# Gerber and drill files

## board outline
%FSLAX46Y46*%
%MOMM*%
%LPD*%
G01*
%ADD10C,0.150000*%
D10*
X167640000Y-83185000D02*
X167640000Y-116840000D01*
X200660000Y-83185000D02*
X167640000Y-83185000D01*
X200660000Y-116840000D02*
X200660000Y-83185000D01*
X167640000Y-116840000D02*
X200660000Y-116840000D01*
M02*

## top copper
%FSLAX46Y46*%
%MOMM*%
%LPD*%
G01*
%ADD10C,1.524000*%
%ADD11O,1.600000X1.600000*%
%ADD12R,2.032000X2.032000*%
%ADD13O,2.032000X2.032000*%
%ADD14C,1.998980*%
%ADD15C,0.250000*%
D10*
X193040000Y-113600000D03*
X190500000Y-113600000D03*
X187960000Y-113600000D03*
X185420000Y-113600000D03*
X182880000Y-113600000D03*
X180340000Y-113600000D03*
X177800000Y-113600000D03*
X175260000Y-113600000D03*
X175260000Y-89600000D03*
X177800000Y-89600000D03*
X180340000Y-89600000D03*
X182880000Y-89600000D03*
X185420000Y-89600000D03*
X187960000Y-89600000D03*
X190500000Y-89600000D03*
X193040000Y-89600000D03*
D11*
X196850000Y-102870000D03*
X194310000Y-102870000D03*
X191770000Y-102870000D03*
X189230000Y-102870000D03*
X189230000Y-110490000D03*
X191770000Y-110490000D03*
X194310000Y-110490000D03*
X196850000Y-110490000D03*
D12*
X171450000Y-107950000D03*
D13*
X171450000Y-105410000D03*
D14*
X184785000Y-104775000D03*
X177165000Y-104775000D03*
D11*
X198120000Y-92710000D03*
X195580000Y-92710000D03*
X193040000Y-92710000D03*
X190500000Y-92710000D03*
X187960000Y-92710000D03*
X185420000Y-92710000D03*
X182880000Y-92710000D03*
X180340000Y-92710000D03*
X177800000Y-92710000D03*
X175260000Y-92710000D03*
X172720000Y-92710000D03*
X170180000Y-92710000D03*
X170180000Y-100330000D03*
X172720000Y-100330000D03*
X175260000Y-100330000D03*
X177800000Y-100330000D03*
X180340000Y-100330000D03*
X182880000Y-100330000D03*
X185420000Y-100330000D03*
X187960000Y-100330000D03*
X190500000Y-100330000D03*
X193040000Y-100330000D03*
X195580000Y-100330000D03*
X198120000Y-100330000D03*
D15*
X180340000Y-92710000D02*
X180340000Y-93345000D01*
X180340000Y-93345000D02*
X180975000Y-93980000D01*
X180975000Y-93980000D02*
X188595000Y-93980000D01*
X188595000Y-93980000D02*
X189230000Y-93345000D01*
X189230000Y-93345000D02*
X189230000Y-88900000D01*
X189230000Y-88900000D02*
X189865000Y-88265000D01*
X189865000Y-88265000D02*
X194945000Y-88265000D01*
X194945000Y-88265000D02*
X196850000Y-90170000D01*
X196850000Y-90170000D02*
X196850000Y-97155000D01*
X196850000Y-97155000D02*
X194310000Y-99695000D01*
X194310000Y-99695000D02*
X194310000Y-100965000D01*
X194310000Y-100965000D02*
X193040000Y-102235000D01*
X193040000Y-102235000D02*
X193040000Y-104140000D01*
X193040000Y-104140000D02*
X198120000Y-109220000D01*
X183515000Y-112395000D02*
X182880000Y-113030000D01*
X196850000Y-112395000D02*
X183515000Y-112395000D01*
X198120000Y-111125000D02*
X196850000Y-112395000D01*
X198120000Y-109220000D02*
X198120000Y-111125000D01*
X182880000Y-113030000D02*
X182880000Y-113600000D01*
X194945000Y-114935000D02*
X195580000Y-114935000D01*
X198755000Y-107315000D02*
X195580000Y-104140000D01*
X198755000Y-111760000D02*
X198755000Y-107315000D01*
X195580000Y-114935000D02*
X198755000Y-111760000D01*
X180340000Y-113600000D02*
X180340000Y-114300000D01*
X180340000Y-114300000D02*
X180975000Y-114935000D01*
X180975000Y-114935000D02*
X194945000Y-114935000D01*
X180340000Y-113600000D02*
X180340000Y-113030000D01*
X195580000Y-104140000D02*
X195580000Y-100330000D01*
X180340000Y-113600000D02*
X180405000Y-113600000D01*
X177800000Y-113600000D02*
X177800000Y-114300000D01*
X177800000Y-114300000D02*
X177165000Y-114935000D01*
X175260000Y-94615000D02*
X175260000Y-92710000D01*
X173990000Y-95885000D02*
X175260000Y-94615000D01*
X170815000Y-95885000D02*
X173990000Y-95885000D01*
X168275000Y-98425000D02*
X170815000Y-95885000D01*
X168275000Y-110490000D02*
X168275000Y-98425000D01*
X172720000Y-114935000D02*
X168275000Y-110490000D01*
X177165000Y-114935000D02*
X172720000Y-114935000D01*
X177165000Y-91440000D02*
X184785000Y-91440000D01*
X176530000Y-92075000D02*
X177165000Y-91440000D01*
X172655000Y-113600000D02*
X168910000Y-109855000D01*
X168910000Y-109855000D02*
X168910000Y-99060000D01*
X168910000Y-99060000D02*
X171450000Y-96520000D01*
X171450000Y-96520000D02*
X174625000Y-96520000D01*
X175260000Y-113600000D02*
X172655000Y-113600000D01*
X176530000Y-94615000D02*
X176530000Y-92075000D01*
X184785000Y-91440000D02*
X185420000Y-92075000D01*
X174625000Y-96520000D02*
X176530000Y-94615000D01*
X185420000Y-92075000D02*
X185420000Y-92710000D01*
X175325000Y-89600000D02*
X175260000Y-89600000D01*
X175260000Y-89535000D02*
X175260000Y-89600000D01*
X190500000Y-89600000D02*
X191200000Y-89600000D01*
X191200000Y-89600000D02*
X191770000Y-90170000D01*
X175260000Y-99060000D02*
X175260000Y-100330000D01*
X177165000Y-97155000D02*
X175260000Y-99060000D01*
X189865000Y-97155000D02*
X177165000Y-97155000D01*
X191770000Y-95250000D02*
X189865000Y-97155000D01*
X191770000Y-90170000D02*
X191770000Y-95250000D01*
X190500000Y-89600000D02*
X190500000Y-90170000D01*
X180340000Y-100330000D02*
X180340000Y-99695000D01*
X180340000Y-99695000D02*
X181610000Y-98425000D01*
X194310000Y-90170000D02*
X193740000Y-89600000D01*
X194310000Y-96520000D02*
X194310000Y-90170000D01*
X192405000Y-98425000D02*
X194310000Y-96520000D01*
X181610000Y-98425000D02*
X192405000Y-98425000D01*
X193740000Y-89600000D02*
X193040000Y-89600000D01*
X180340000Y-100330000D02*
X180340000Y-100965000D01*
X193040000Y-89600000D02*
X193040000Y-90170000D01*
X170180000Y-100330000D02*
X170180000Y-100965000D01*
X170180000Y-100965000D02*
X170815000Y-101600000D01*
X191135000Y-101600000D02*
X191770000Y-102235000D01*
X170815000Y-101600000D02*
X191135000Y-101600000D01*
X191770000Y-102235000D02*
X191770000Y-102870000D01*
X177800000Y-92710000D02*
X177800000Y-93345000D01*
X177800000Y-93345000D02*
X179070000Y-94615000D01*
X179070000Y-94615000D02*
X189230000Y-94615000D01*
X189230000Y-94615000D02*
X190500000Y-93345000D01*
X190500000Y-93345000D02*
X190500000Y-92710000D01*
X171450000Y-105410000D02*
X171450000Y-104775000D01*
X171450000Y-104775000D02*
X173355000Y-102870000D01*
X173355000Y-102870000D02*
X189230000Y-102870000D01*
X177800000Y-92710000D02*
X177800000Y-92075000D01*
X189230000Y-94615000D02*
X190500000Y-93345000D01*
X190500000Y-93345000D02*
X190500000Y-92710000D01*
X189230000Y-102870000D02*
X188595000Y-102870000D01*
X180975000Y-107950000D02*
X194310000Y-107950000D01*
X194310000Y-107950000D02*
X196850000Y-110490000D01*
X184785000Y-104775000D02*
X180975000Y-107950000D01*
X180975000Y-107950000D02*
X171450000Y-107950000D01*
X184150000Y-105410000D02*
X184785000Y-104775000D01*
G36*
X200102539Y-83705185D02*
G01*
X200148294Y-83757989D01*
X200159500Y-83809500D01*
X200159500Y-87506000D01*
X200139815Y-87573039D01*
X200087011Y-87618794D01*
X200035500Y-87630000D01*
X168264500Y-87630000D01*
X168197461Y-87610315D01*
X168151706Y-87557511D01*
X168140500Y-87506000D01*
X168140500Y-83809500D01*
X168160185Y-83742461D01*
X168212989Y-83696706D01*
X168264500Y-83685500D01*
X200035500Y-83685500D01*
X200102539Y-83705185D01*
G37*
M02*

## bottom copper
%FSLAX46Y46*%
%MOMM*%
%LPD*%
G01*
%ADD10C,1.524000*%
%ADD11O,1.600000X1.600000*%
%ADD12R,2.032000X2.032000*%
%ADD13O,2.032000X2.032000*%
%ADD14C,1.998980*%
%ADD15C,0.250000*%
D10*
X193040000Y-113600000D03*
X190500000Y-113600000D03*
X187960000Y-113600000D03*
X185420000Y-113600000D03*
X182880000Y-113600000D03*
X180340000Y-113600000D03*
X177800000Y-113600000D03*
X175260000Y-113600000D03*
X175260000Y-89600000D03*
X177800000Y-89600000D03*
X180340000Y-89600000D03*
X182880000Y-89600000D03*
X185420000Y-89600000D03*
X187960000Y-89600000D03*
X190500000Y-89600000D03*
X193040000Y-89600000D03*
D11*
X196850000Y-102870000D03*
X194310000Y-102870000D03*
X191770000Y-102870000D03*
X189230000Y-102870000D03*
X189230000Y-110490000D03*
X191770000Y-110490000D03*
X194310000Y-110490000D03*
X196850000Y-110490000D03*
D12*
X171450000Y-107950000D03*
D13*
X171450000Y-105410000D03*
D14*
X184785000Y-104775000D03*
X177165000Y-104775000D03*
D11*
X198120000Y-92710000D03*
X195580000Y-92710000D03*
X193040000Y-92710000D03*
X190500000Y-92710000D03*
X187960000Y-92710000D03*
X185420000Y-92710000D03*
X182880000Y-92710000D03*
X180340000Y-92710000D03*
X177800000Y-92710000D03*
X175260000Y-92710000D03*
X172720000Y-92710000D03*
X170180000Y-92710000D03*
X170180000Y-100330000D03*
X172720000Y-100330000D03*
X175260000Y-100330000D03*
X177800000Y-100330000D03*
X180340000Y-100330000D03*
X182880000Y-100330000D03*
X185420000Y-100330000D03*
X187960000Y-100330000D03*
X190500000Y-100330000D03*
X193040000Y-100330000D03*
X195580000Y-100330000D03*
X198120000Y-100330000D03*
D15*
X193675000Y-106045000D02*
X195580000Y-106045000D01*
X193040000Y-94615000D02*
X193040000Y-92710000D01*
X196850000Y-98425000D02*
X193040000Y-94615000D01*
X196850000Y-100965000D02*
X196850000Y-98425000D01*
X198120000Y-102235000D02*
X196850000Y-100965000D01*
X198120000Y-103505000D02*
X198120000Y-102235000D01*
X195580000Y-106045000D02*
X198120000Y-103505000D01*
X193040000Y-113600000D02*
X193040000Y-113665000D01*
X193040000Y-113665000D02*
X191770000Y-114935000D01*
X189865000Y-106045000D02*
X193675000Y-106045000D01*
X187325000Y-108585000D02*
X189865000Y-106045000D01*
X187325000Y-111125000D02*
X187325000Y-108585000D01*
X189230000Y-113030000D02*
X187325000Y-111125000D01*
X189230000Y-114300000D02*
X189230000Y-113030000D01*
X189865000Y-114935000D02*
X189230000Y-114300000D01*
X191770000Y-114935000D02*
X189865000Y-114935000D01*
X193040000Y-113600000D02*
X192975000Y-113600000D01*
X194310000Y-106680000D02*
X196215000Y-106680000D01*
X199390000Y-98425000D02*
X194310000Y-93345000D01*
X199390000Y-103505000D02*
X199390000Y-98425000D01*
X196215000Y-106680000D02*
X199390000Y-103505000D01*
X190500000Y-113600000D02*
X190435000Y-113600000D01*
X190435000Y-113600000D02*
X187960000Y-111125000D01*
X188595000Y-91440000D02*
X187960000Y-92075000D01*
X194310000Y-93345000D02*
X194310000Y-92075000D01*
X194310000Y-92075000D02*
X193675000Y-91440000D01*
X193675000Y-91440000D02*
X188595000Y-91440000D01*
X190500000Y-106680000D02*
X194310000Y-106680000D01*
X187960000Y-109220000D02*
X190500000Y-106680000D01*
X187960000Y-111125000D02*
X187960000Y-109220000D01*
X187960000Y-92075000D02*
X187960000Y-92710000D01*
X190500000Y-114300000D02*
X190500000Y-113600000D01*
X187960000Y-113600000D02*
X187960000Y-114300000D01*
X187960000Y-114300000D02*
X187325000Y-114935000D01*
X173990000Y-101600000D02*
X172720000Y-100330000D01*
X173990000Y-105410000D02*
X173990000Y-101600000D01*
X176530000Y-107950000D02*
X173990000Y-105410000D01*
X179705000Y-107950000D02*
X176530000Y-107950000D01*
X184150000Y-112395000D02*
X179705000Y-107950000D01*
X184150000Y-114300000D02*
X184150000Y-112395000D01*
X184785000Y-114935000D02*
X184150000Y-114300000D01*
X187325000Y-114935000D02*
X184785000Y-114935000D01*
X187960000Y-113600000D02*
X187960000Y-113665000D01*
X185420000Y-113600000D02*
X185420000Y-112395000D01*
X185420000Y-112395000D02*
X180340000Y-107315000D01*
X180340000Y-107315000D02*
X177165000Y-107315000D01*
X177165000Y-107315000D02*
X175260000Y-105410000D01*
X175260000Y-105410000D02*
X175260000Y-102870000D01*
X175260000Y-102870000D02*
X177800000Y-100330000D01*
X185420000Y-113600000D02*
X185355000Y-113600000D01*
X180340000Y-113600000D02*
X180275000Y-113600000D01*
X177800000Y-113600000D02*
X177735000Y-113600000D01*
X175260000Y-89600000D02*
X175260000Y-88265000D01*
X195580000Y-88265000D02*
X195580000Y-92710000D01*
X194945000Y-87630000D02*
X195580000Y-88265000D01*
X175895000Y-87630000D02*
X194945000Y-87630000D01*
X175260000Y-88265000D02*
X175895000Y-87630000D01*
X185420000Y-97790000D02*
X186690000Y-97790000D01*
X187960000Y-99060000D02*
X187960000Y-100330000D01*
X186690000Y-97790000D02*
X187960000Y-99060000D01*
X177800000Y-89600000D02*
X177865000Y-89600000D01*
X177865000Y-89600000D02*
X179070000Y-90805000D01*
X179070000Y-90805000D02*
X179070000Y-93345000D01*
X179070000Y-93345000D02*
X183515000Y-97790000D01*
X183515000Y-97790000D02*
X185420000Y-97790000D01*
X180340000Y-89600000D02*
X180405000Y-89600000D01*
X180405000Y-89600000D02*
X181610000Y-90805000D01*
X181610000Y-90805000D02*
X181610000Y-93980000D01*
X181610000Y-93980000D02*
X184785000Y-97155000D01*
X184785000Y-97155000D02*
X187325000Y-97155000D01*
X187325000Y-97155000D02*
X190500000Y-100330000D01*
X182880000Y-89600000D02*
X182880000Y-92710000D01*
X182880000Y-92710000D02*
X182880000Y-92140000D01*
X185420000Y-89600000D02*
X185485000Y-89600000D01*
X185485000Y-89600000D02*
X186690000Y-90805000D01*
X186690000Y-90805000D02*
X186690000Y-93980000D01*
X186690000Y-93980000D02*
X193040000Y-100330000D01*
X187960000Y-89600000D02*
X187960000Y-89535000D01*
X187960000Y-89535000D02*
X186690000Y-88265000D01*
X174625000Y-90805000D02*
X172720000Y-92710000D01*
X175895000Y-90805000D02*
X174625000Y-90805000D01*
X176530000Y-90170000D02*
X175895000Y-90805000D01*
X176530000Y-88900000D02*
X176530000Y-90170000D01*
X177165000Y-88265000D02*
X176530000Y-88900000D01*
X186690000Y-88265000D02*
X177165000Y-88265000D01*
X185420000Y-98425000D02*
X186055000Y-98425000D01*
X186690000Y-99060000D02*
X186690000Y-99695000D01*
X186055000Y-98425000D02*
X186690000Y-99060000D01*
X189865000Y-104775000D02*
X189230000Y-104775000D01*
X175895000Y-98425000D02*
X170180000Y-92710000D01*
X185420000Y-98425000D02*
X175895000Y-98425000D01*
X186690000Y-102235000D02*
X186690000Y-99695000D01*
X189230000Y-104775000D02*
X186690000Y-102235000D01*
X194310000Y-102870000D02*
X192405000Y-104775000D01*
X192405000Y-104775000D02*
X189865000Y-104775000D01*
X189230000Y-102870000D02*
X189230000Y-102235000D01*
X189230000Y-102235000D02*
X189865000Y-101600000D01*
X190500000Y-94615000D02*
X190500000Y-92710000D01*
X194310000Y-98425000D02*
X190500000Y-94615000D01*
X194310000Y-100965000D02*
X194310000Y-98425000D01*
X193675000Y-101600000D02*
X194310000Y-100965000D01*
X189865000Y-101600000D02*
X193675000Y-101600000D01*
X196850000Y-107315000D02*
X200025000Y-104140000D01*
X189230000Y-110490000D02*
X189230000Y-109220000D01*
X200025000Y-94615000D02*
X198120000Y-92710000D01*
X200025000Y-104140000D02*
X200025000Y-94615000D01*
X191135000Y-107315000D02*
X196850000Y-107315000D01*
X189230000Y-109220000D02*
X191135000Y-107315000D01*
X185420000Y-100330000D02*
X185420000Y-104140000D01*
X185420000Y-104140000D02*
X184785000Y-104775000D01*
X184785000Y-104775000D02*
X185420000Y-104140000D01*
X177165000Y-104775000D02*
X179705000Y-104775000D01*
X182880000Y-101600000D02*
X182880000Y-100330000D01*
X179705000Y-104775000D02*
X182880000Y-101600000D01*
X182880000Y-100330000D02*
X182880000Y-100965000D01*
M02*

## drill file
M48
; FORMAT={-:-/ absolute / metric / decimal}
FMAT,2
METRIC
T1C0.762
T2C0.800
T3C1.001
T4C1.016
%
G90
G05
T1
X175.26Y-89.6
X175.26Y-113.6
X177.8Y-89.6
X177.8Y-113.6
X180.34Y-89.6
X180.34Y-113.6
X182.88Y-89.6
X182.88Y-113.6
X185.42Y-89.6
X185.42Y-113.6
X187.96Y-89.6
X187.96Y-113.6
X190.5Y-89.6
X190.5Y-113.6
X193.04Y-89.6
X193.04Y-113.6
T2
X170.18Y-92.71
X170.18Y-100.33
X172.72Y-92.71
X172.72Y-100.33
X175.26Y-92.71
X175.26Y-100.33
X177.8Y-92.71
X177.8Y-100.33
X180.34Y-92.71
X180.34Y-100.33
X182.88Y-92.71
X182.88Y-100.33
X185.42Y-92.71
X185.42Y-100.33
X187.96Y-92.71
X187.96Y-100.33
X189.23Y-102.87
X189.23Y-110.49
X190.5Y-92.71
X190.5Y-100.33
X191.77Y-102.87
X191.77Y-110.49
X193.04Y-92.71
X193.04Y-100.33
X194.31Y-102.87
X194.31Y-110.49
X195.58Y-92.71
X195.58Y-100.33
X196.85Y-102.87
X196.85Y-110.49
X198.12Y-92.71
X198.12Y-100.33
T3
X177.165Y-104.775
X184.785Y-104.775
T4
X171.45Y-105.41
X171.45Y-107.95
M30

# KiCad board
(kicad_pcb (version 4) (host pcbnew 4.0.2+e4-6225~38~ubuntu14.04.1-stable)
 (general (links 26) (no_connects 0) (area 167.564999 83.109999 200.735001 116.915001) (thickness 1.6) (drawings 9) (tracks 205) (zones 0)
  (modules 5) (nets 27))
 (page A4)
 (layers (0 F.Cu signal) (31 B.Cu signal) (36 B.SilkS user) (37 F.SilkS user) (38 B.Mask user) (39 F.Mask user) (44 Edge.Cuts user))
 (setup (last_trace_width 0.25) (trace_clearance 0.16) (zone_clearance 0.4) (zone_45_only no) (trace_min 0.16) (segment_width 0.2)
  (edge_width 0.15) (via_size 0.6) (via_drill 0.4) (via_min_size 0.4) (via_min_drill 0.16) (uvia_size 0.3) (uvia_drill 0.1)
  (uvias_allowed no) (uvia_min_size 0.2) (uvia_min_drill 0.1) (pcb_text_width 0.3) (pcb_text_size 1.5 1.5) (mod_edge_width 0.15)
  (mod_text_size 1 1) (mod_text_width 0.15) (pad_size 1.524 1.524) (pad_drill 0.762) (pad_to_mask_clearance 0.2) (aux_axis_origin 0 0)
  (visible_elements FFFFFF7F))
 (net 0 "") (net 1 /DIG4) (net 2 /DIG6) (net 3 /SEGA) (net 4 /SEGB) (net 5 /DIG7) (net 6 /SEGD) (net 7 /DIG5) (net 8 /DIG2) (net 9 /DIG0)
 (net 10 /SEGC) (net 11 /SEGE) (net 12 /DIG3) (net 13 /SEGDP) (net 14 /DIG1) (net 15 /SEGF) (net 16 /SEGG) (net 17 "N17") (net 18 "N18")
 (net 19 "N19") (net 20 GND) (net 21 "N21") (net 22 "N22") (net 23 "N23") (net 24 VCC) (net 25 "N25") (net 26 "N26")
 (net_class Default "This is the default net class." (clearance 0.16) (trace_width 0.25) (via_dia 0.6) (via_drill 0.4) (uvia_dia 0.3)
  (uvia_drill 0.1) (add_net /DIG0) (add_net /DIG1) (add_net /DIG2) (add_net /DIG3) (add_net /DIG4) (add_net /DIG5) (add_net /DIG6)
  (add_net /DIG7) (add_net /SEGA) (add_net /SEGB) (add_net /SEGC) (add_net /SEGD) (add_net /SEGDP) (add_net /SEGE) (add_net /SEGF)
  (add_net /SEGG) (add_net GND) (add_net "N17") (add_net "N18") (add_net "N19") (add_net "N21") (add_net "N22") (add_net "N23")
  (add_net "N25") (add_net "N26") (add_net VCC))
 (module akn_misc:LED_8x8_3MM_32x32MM (layer B.Cu) (at 184.15 101.6 90)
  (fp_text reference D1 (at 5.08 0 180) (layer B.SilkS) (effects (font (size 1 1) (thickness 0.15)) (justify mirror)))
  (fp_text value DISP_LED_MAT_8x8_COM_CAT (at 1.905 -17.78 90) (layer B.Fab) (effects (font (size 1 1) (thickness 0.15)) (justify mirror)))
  (pad 1 thru_hole circle (at -12 8.89 90) (size 1.524 1.524) (drill 0.762) (layers *.Cu *.Mask B.SilkS) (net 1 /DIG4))
  (pad 2 thru_hole circle (at -12 6.35 90) (size 1.524 1.524) (drill 0.762) (layers *.Cu *.Mask B.SilkS) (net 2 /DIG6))
  (pad 3 thru_hole circle (at -12 3.81 90) (size 1.524 1.524) (drill 0.762) (layers *.Cu *.Mask B.SilkS) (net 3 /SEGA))
  (pad 4 thru_hole circle (at -12 1.27 90) (size 1.524 1.524) (drill 0.762) (layers *.Cu *.Mask B.SilkS) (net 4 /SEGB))
  (pad 5 thru_hole circle (at -12 -1.27 90) (size 1.524 1.524) (drill 0.762) (layers *.Cu *.Mask B.SilkS) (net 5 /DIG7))
  (pad 6 thru_hole circle (at -12 -3.81 90) (size 1.524 1.524) (drill 0.762) (layers *.Cu *.Mask B.SilkS) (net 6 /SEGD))
  (pad 7 thru_hole circle (at -12 -6.35 90) (size 1.524 1.524) (drill 0.762) (layers *.Cu *.Mask B.SilkS) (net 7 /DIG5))
  (pad 8 thru_hole circle (at -12 -8.89 90) (size 1.524 1.524) (drill 0.762) (layers *.Cu *.Mask B.SilkS) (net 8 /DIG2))
  (pad 9 thru_hole circle (at 12 -8.89 90) (size 1.524 1.524) (drill 0.762) (layers *.Cu *.Mask B.SilkS) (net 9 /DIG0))
  (pad 10 thru_hole circle (at 12 -6.35 90) (size 1.524 1.524) (drill 0.762) (layers *.Cu *.Mask B.SilkS) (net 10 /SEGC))
  (pad 11 thru_hole circle (at 12 -3.81 90) (size 1.524 1.524) (drill 0.762) (layers *.Cu *.Mask B.SilkS) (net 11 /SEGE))
  (pad 12 thru_hole circle (at 12 -1.27 90) (size 1.524 1.524) (drill 0.762) (layers *.Cu *.Mask B.SilkS) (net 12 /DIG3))
  (pad 13 thru_hole circle (at 12 1.27 90) (size 1.524 1.524) (drill 0.762) (layers *.Cu *.Mask B.SilkS) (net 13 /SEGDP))
  (pad 14 thru_hole circle (at 12 3.81 90) (size 1.524 1.524) (drill 0.762) (layers *.Cu *.Mask B.SilkS) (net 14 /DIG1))
  (pad 15 thru_hole circle (at 12 6.35 90) (size 1.524 1.524) (drill 0.762) (layers *.Cu *.Mask B.SilkS) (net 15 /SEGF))
  (pad 16 thru_hole circle (at 12 8.89 90) (size 1.524 1.524) (drill 0.762) (layers *.Cu *.Mask B.SilkS) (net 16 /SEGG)))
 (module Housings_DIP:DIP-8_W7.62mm (layer F.Cu) (at 196.85 102.87 270)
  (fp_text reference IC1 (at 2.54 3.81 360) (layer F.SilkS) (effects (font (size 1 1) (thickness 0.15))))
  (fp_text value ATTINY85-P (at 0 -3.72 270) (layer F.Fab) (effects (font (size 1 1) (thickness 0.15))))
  (pad 1 thru_hole oval (at 0 0 270) (size 1.6 1.6) (drill 0.8) (layers *.Cu *.Mask F.SilkS) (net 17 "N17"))
  (pad 2 thru_hole oval (at 0 2.54 270) (size 1.6 1.6) (drill 0.8) (layers *.Cu *.Mask F.SilkS) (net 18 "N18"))
  (pad 3 thru_hole oval (at 0 5.08 270) (size 1.6 1.6) (drill 0.8) (layers *.Cu *.Mask F.SilkS) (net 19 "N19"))
  (pad 4 thru_hole oval (at 0 7.62 270) (size 1.6 1.6) (drill 0.8) (layers *.Cu *.Mask F.SilkS) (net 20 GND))
  (pad 5 thru_hole oval (at 7.62 7.62 270) (size 1.6 1.6) (drill 0.8) (layers *.Cu *.Mask F.SilkS) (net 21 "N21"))
  (pad 6 thru_hole oval (at 7.62 5.08 270) (size 1.6 1.6) (drill 0.8) (layers *.Cu *.Mask F.SilkS) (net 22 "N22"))
  (pad 7 thru_hole oval (at 7.62 2.54 270) (size 1.6 1.6) (drill 0.8) (layers *.Cu *.Mask F.SilkS) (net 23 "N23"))
  (pad 8 thru_hole oval (at 7.62 0 270) (size 1.6 1.6) (drill 0.8) (layers *.Cu *.Mask F.SilkS) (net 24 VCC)))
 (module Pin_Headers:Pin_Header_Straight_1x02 (layer F.Cu) (at 171.45 107.95 180)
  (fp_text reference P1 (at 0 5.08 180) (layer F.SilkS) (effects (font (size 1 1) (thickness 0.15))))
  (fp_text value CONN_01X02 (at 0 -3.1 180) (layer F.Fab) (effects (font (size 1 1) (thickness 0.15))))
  (pad 1 thru_hole rect (at 0 0 180) (size 2.032 2.032) (drill 1.016) (layers *.Cu *.Mask F.SilkS) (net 24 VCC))
  (pad 2 thru_hole oval (at 0 2.54 180) (size 2.032 2.032) (drill 1.016) (layers *.Cu *.Mask F.SilkS) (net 20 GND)))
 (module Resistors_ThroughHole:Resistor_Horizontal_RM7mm (layer F.Cu) (at 184.785 104.775 180)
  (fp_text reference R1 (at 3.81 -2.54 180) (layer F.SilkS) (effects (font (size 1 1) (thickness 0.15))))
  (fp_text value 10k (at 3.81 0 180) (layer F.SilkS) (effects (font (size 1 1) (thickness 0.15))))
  (pad 1 thru_hole circle (at 0 0 180) (size 1.99898 1.99898) (drill 1.00076) (layers *.Cu *.SilkS *.Mask) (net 24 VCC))
  (pad 2 thru_hole circle (at 7.62 0 180) (size 1.99898 1.99898) (drill 1.00076) (layers *.Cu *.SilkS *.Mask) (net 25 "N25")))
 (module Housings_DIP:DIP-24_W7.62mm (layer F.Cu) (at 198.12 92.71 270)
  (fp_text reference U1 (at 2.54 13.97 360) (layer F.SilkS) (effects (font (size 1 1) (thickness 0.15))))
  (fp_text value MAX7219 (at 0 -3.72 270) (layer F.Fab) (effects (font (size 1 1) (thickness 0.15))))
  (pad 1 thru_hole oval (at 0 0 270) (size 1.6 1.6) (drill 0.8) (layers *.Cu *.Mask F.SilkS) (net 21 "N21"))
  (pad 2 thru_hole oval (at 0 2.54 270) (size 1.6 1.6) (drill 0.8) (layers *.Cu *.Mask F.SilkS) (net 9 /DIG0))
  (pad 3 thru_hole oval (at 0 5.08 270) (size 1.6 1.6) (drill 0.8) (layers *.Cu *.Mask F.SilkS) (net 1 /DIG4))
  (pad 4 thru_hole oval (at 0 7.62 270) (size 1.6 1.6) (drill 0.8) (layers *.Cu *.Mask F.SilkS) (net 20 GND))
  (pad 5 thru_hole oval (at 0 10.16 270) (size 1.6 1.6) (drill 0.8) (layers *.Cu *.Mask F.SilkS) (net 2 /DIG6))
  (pad 6 thru_hole oval (at 0 12.7 270) (size 1.6 1.6) (drill 0.8) (layers *.Cu *.Mask F.SilkS) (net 8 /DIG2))
  (pad 7 thru_hole oval (at 0 15.24 270) (size 1.6 1.6) (drill 0.8) (layers *.Cu *.Mask F.SilkS) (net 12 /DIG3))
  (pad 8 thru_hole oval (at 0 17.78 270) (size 1.6 1.6) (drill 0.8) (layers *.Cu *.Mask F.SilkS) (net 5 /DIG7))
  (pad 9 thru_hole oval (at 0 20.32 270) (size 1.6 1.6) (drill 0.8) (layers *.Cu *.Mask F.SilkS) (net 20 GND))
  (pad 10 thru_hole oval (at 0 22.86 270) (size 1.6 1.6) (drill 0.8) (layers *.Cu *.Mask F.SilkS) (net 7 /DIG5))
  (pad 11 thru_hole oval (at 0 25.4 270) (size 1.6 1.6) (drill 0.8) (layers *.Cu *.Mask F.SilkS) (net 14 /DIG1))
  (pad 12 thru_hole oval (at 0 27.94 270) (size 1.6 1.6) (drill 0.8) (layers *.Cu *.Mask F.SilkS) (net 18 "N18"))
  (pad 13 thru_hole oval (at 7.62 27.94 270) (size 1.6 1.6) (drill 0.8) (layers *.Cu *.Mask F.SilkS) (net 19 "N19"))
  (pad 14 thru_hole oval (at 7.62 25.4 270) (size 1.6 1.6) (drill 0.8) (layers *.Cu *.Mask F.SilkS) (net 3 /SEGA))
  (pad 15 thru_hole oval (at 7.62 22.86 270) (size 1.6 1.6) (drill 0.8) (layers *.Cu *.Mask F.SilkS) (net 15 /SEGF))
  (pad 16 thru_hole oval (at 7.62 20.32 270) (size 1.6 1.6) (drill 0.8) (layers *.Cu *.Mask F.SilkS) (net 4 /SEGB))
  (pad 17 thru_hole oval (at 7.62 17.78 270) (size 1.6 1.6) (drill 0.8) (layers *.Cu *.Mask F.SilkS) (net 16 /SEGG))
  (pad 18 thru_hole oval (at 7.62 15.24 270) (size 1.6 1.6) (drill 0.8) (layers *.Cu *.Mask F.SilkS) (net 25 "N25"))
  (pad 19 thru_hole oval (at 7.62 12.7 270) (size 1.6 1.6) (drill 0.8) (layers *.Cu *.Mask F.SilkS) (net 24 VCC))
  (pad 20 thru_hole oval (at 7.62 10.16 270) (size 1.6 1.6) (drill 0.8) (layers *.Cu *.Mask F.SilkS) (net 10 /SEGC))
  (pad 21 thru_hole oval (at 7.62 7.62 270) (size 1.6 1.6) (drill 0.8) (layers *.Cu *.Mask F.SilkS) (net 11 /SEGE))
  (pad 22 thru_hole oval (at 7.62 5.08 270) (size 1.6 1.6) (drill 0.8) (layers *.Cu *.Mask F.SilkS) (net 13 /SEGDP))
  (pad 23 thru_hole oval (at 7.62 2.54 270) (size 1.6 1.6) (drill 0.8) (layers *.Cu *.Mask F.SilkS) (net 6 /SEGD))
  (pad 24 thru_hole oval (at 7.62 0 270) (size 1.6 1.6) (drill 0.8) (layers *.Cu *.Mask F.SilkS) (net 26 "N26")))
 (gr_line (start 167.64 83.185) (end 167.64 116.84) (angle 90) (layer Edge.Cuts) (width 0.15))
 (gr_line (start 200.66 83.185) (end 167.64 83.185) (angle 90) (layer Edge.Cuts) (width 0.15))
 (gr_line (start 200.66 116.84) (end 200.66 83.185) (angle 90) (layer Edge.Cuts) (width 0.15))
 (gr_line (start 167.64 116.84) (end 200.66 116.84) (angle 90) (layer Edge.Cuts) (width 0.15))
 (segment (start 193.675 106.045) (end 195.58 106.045) (width 0.25) (layer B.Cu) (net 1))
 (segment (start 193.04 94.615) (end 193.04 92.71) (width 0.25) (layer B.Cu) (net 1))
 (segment (start 196.85 98.425) (end 193.04 94.615) (width 0.25) (layer B.Cu) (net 1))
 (segment (start 196.85 100.965) (end 196.85 98.425) (width 0.25) (layer B.Cu) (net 1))
 (segment (start 198.12 102.235) (end 196.85 100.965) (width 0.25) (layer B.Cu) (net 1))
 (segment (start 198.12 103.505) (end 198.12 102.235) (width 0.25) (layer B.Cu) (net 1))
 (segment (start 195.58 106.045) (end 198.12 103.505) (width 0.25) (layer B.Cu) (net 1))
 (segment (start 193.04 113.6) (end 193.04 113.665) (width 0.25) (layer B.Cu) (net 1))
 (segment (start 193.04 113.665) (end 191.77 114.935) (width 0.25) (layer B.Cu) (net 1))
 (segment (start 189.865 106.045) (end 193.675 106.045) (width 0.25) (layer B.Cu) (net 1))
 (segment (start 187.325 108.585) (end 189.865 106.045) (width 0.25) (layer B.Cu) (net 1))
 (segment (start 187.325 111.125) (end 187.325 108.585) (width 0.25) (layer B.Cu) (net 1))
 (segment (start 189.23 113.03) (end 187.325 111.125) (width 0.25) (layer B.Cu) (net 1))
 (segment (start 189.23 114.3) (end 189.23 113.03) (width 0.25) (layer B.Cu) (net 1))
 (segment (start 189.865 114.935) (end 189.23 114.3) (width 0.25) (layer B.Cu) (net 1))
 (segment (start 191.77 114.935) (end 189.865 114.935) (width 0.25) (layer B.Cu) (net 1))
 (segment (start 193.04 113.6) (end 192.975 113.6) (width 0.25) (layer B.Cu) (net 1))
 (segment (start 194.31 106.68) (end 196.215 106.68) (width 0.25) (layer B.Cu) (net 2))
 (segment (start 199.39 98.425) (end 194.31 93.345) (width 0.25) (layer B.Cu) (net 2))
 (segment (start 199.39 103.505) (end 199.39 98.425) (width 0.25) (layer B.Cu) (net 2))
 (segment (start 196.215 106.68) (end 199.39 103.505) (width 0.25) (layer B.Cu) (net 2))
 (segment (start 190.5 113.6) (end 190.435 113.6) (width 0.25) (layer B.Cu) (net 2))
 (segment (start 190.435 113.6) (end 187.96 111.125) (width 0.25) (layer B.Cu) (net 2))
 (segment (start 188.595 91.44) (end 187.96 92.075) (width 0.25) (layer B.Cu) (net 2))
 (segment (start 194.31 93.345) (end 194.31 92.075) (width 0.25) (layer B.Cu) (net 2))
 (segment (start 194.31 92.075) (end 193.675 91.44) (width 0.25) (layer B.Cu) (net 2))
 (segment (start 193.675 91.44) (end 188.595 91.44) (width 0.25) (layer B.Cu) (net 2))
 (segment (start 190.5 106.68) (end 194.31 106.68) (width 0.25) (layer B.Cu) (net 2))
 (segment (start 187.96 109.22) (end 190.5 106.68) (width 0.25) (layer B.Cu) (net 2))
 (segment (start 187.96 111.125) (end 187.96 109.22) (width 0.25) (layer B.Cu) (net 2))
 (segment (start 187.96 92.075) (end 187.96 92.71) (width 0.25) (layer B.Cu) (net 2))
 (segment (start 190.5 114.3) (end 190.5 113.6) (width 0.25) (layer B.Cu) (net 2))
 (segment (start 187.96 113.6) (end 187.96 114.3) (width 0.25) (layer B.Cu) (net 3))
 (segment (start 187.96 114.3) (end 187.325 114.935) (width 0.25) (layer B.Cu) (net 3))
 (segment (start 173.99 101.6) (end 172.72 100.33) (width 0.25) (layer B.Cu) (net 3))
 (segment (start 173.99 105.41) (end 173.99 101.6) (width 0.25) (layer B.Cu) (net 3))
 (segment (start 176.53 107.95) (end 173.99 105.41) (width 0.25) (layer B.Cu) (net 3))
 (segment (start 179.705 107.95) (end 176.53 107.95) (width 0.25) (layer B.Cu) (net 3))
 (segment (start 184.15 112.395) (end 179.705 107.95) (width 0.25) (layer B.Cu) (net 3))
 (segment (start 184.15 114.3) (end 184.15 112.395) (width 0.25) (layer B.Cu) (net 3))
 (segment (start 184.785 114.935) (end 184.15 114.3) (width 0.25) (layer B.Cu) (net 3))
 (segment (start 187.325 114.935) (end 184.785 114.935) (width 0.25) (layer B.Cu) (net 3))
 (segment (start 187.96 113.6) (end 187.96 113.665) (width 0.25) (layer B.Cu) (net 3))
 (segment (start 185.42 113.6) (end 185.42 112.395) (width 0.25) (layer B.Cu) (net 4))
 (segment (start 185.42 112.395) (end 180.34 107.315) (width 0.25) (layer B.Cu) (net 4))
 (segment (start 180.34 107.315) (end 177.165 107.315) (width 0.25) (layer B.Cu) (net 4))
 (segment (start 177.165 107.315) (end 175.26 105.41) (width 0.25) (layer B.Cu) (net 4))
 (segment (start 175.26 105.41) (end 175.26 102.87) (width 0.25) (layer B.Cu) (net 4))
 (segment (start 175.26 102.87) (end 177.8 100.33) (width 0.25) (layer B.Cu) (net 4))
 (segment (start 185.42 113.6) (end 185.355 113.6) (width 0.25) (layer B.Cu) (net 4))
 (segment (start 180.34 92.71) (end 180.34 93.345) (width 0.25) (layer F.Cu) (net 5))
 (segment (start 180.34 93.345) (end 180.975 93.98) (width 0.25) (layer F.Cu) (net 5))
 (segment (start 180.975 93.98) (end 188.595 93.98) (width 0.25) (layer F.Cu) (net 5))
 (segment (start 188.595 93.98) (end 189.23 93.345) (width 0.25) (layer F.Cu) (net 5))
 (segment (start 189.23 93.345) (end 189.23 88.9) (width 0.25) (layer F.Cu) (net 5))
 (segment (start 189.23 88.9) (end 189.865 88.265) (width 0.25) (layer F.Cu) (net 5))
 (segment (start 189.865 88.265) (end 194.945 88.265) (width 0.25) (layer F.Cu) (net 5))
 (segment (start 194.945 88.265) (end 196.85 90.17) (width 0.25) (layer F.Cu) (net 5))
 (segment (start 196.85 90.17) (end 196.85 97.155) (width 0.25) (layer F.Cu) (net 5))
 (segment (start 196.85 97.155) (end 194.31 99.695) (width 0.25) (layer F.Cu) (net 5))
 (segment (start 194.31 99.695) (end 194.31 100.965) (width 0.25) (layer F.Cu) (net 5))
 (segment (start 194.31 100.965) (end 193.04 102.235) (width 0.25) (layer F.Cu) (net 5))
 (segment (start 193.04 102.235) (end 193.04 104.14) (width 0.25) (layer F.Cu) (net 5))
 (segment (start 193.04 104.14) (end 198.12 109.22) (width 0.25) (layer F.Cu) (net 5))
 (segment (start 183.515 112.395) (end 182.88 113.03) (width 0.25) (layer F.Cu) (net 5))
 (segment (start 196.85 112.395) (end 183.515 112.395) (width 0.25) (layer F.Cu) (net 5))
 (segment (start 198.12 111.125) (end 196.85 112.395) (width 0.25) (layer F.Cu) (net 5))
 (segment (start 198.12 109.22) (end 198.12 111.125) (width 0.25) (layer F.Cu) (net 5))
 (segment (start 182.88 113.03) (end 182.88 113.6) (width 0.25) (layer F.Cu) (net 5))
 (segment (start 180.34 113.6) (end 180.275 113.6) (width 0.25) (layer B.Cu) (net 6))
 (segment (start 194.945 114.935) (end 195.58 114.935) (width 0.25) (layer F.Cu) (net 6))
 (segment (start 198.755 107.315) (end 195.58 104.14) (width 0.25) (layer F.Cu) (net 6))
 (segment (start 198.755 111.76) (end 198.755 107.315) (width 0.25) (layer F.Cu) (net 6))
 (segment (start 195.58 114.935) (end 198.755 111.76) (width 0.25) (layer F.Cu) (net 6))
 (segment (start 180.34 113.6) (end 180.34 114.3) (width 0.25) (layer F.Cu) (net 6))
 (segment (start 180.34 114.3) (end 180.975 114.935) (width 0.25) (layer F.Cu) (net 6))
 (segment (start 180.975 114.935) (end 194.945 114.935) (width 0.25) (layer F.Cu) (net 6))
 (segment (start 180.34 113.6) (end 180.34 113.03) (width 0.25) (layer F.Cu) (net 6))
 (segment (start 195.58 104.14) (end 195.58 100.33) (width 0.25) (layer F.Cu) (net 6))
 (segment (start 180.34 113.6) (end 180.405 113.6) (width 0.25) (layer F.Cu) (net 6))
 (segment (start 177.8 113.6) (end 177.735 113.6) (width 0.25) (layer B.Cu) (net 7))
 (segment (start 177.8 113.6) (end 177.8 114.3) (width 0.25) (layer F.Cu) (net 7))
 (segment (start 177.8 114.3) (end 177.165 114.935) (width 0.25) (layer F.Cu) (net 7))
 (segment (start 175.26 94.615) (end 175.26 92.71) (width 0.25) (layer F.Cu) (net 7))
 (segment (start 173.99 95.885) (end 175.26 94.615) (width 0.25) (layer F.Cu) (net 7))
 (segment (start 170.815 95.885) (end 173.99 95.885) (width 0.25) (layer F.Cu) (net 7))
 (segment (start 168.275 98.425) (end 170.815 95.885) (width 0.25) (layer F.Cu) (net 7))
 (segment (start 168.275 110.49) (end 168.275 98.425) (width 0.25) (layer F.Cu) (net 7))
 (segment (start 172.72 114.935) (end 168.275 110.49) (width 0.25) (layer F.Cu) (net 7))
 (segment (start 177.165 114.935) (end 172.72 114.935) (width 0.25) (layer F.Cu) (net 7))
 (segment (start 177.165 91.44) (end 184.785 91.44) (width 0.25) (layer F.Cu) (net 8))
 (segment (start 176.53 92.075) (end 177.165 91.44) (width 0.25) (layer F.Cu) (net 8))
 (segment (start 172.655 113.6) (end 168.91 109.855) (width 0.25) (layer F.Cu) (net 8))
 (segment (start 168.91 109.855) (end 168.91 99.06) (width 0.25) (layer F.Cu) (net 8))
 (segment (start 168.91 99.06) (end 171.45 96.52) (width 0.25) (layer F.Cu) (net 8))
 (segment (start 171.45 96.52) (end 174.625 96.52) (width 0.25) (layer F.Cu) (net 8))
 (segment (start 175.26 113.6) (end 172.655 113.6) (width 0.25) (layer F.Cu) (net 8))
 (segment (start 176.53 94.615) (end 176.53 92.075) (width 0.25) (layer F.Cu) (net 8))
 (segment (start 184.785 91.44) (end 185.42 92.075) (width 0.25) (layer F.Cu) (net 8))
 (segment (start 174.625 96.52) (end 176.53 94.615) (width 0.25) (layer F.Cu) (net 8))
 (segment (start 185.42 92.075) (end 185.42 92.71) (width 0.25) (layer F.Cu) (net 8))
 (segment (start 175.325 89.6) (end 175.26 89.6) (width 0.25) (layer F.Cu) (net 9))
 (segment (start 175.26 89.535) (end 175.26 89.6) (width 0.25) (layer F.Cu) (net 9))
 (segment (start 175.26 89.6) (end 175.26 88.265) (width 0.25) (layer B.Cu) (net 9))
 (segment (start 195.58 88.265) (end 195.58 92.71) (width 0.25) (layer B.Cu) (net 9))
 (segment (start 194.945 87.63) (end 195.58 88.265) (width 0.25) (layer B.Cu) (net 9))
 (segment (start 175.895 87.63) (end 194.945 87.63) (width 0.25) (layer B.Cu) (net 9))
 (segment (start 175.26 88.265) (end 175.895 87.63) (width 0.25) (layer B.Cu) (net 9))
 (segment (start 185.42 97.79) (end 186.69 97.79) (width 0.25) (layer B.Cu) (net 10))
 (segment (start 187.96 99.06) (end 187.96 100.33) (width 0.25) (layer B.Cu) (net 10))
 (segment (start 186.69 97.79) (end 187.96 99.06) (width 0.25) (layer B.Cu) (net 10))
 (segment (start 177.8 89.6) (end 177.865 89.6) (width 0.25) (layer B.Cu) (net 10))
 (segment (start 177.865 89.6) (end 179.07 90.805) (width 0.25) (layer B.Cu) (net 10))
 (segment (start 179.07 90.805) (end 179.07 93.345) (width 0.25) (layer B.Cu) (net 10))
 (segment (start 179.07 93.345) (end 183.515 97.79) (width 0.25) (layer B.Cu) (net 10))
 (segment (start 183.515 97.79) (end 185.42 97.79) (width 0.25) (layer B.Cu) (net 10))
 (segment (start 180.34 89.6) (end 180.405 89.6) (width 0.25) (layer B.Cu) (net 11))
 (segment (start 180.405 89.6) (end 181.61 90.805) (width 0.25) (layer B.Cu) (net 11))
 (segment (start 181.61 90.805) (end 181.61 93.98) (width 0.25) (layer B.Cu) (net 11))
 (segment (start 181.61 93.98) (end 184.785 97.155) (width 0.25) (layer B.Cu) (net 11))
 (segment (start 184.785 97.155) (end 187.325 97.155) (width 0.25) (layer B.Cu) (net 11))
 (segment (start 187.325 97.155) (end 190.5 100.33) (width 0.25) (layer B.Cu) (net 11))
 (segment (start 182.88 89.6) (end 182.88 92.71) (width 0.25) (layer B.Cu) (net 12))
 (segment (start 182.88 92.71) (end 182.88 92.14) (width 0.25) (layer B.Cu) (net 12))
 (segment (start 185.42 89.6) (end 185.485 89.6) (width 0.25) (layer B.Cu) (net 13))
 (segment (start 185.485 89.6) (end 186.69 90.805) (width 0.25) (layer B.Cu) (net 13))
 (segment (start 186.69 90.805) (end 186.69 93.98) (width 0.25) (layer B.Cu) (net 13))
 (segment (start 186.69 93.98) (end 193.04 100.33) (width 0.25) (layer B.Cu) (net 13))
 (segment (start 187.96 89.6) (end 187.96 89.535) (width 0.25) (layer B.Cu) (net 14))
 (segment (start 187.96 89.535) (end 186.69 88.265) (width 0.25) (layer B.Cu) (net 14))
 (segment (start 174.625 90.805) (end 172.72 92.71) (width 0.25) (layer B.Cu) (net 14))
 (segment (start 175.895 90.805) (end 174.625 90.805) (width 0.25) (layer B.Cu) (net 14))
 (segment (start 176.53 90.17) (end 175.895 90.805) (width 0.25) (layer B.Cu) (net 14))
 (segment (start 176.53 88.9) (end 176.53 90.17) (width 0.25) (layer B.Cu) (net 14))
 (segment (start 177.165 88.265) (end 176.53 88.9) (width 0.25) (layer B.Cu) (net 14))
 (segment (start 186.69 88.265) (end 177.165 88.265) (width 0.25) (layer B.Cu) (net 14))
 (segment (start 190.5 89.6) (end 191.2 89.6) (width 0.25) (layer F.Cu) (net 15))
 (segment (start 191.2 89.6) (end 191.77 90.17) (width 0.25) (layer F.Cu) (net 15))
 (segment (start 175.26 99.06) (end 175.26 100.33) (width 0.25) (layer F.Cu) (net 15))
 (segment (start 177.165 97.155) (end 175.26 99.06) (width 0.25) (layer F.Cu) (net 15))
 (segment (start 189.865 97.155) (end 177.165 97.155) (width 0.25) (layer F.Cu) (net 15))
 (segment (start 191.77 95.25) (end 189.865 97.155) (width 0.25) (layer F.Cu) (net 15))
 (segment (start 191.77 90.17) (end 191.77 95.25) (width 0.25) (layer F.Cu) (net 15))
 (segment (start 190.5 89.6) (end 190.5 90.17) (width 0.25) (layer F.Cu) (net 15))
 (segment (start 180.34 100.33) (end 180.34 99.695) (width 0.25) (layer F.Cu) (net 16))
 (segment (start 180.34 99.695) (end 181.61 98.425) (width 0.25) (layer F.Cu) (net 16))
 (segment (start 194.31 90.17) (end 193.74 89.6) (width 0.25) (layer F.Cu) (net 16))
 (segment (start 194.31 96.52) (end 194.31 90.17) (width 0.25) (layer F.Cu) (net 16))
 (segment (start 192.405 98.425) (end 194.31 96.52) (width 0.25) (layer F.Cu) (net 16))
 (segment (start 181.61 98.425) (end 192.405 98.425) (width 0.25) (layer F.Cu) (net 16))
 (segment (start 193.74 89.6) (end 193.04 89.6) (width 0.25) (layer F.Cu) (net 16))
 (segment (start 180.34 100.33) (end 180.34 100.965) (width 0.25) (layer F.Cu) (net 16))
 (segment (start 193.04 89.6) (end 193.04 90.17) (width 0.25) (layer F.Cu) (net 16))
 (segment (start 185.42 98.425) (end 186.055 98.425) (width 0.25) (layer B.Cu) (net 18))
 (segment (start 186.69 99.06) (end 186.69 99.695) (width 0.25) (layer B.Cu) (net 18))
 (segment (start 186.055 98.425) (end 186.69 99.06) (width 0.25) (layer B.Cu) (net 18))
 (segment (start 189.865 104.775) (end 189.23 104.775) (width 0.25) (layer B.Cu) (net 18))
 (segment (start 175.895 98.425) (end 170.18 92.71) (width 0.25) (layer B.Cu) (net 18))
 (segment (start 185.42 98.425) (end 175.895 98.425) (width 0.25) (layer B.Cu) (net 18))
 (segment (start 186.69 102.235) (end 186.69 99.695) (width 0.25) (layer B.Cu) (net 18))
 (segment (start 189.23 104.775) (end 186.69 102.235) (width 0.25) (layer B.Cu) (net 18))
 (segment (start 194.31 102.87) (end 192.405 104.775) (width 0.25) (layer B.Cu) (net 18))
 (segment (start 192.405 104.775) (end 189.865 104.775) (width 0.25) (layer B.Cu) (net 18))
 (segment (start 170.18 100.33) (end 170.18 100.965) (width 0.25) (layer F.Cu) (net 19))
 (segment (start 170.18 100.965) (end 170.815 101.6) (width 0.25) (layer F.Cu) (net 19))
 (segment (start 191.135 101.6) (end 191.77 102.235) (width 0.25) (layer F.Cu) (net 19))
 (segment (start 170.815 101.6) (end 191.135 101.6) (width 0.25) (layer F.Cu) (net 19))
 (segment (start 191.77 102.235) (end 191.77 102.87) (width 0.25) (layer F.Cu) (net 19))
 (segment (start 177.8 92.71) (end 177.8 93.345) (width 0.25) (layer F.Cu) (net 20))
 (segment (start 177.8 93.345) (end 179.07 94.615) (width 0.25) (layer F.Cu) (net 20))
 (segment (start 179.07 94.615) (end 189.23 94.615) (width 0.25) (layer F.Cu) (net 20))
 (segment (start 189.23 94.615) (end 190.5 93.345) (width 0.25) (layer F.Cu) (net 20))
 (segment (start 190.5 93.345) (end 190.5 92.71) (width 0.25) (layer F.Cu) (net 20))
 (segment (start 189.23 102.87) (end 189.23 102.235) (width 0.25) (layer B.Cu) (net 20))
 (segment (start 189.23 102.235) (end 189.865 101.6) (width 0.25) (layer B.Cu) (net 20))
 (segment (start 190.5 94.615) (end 190.5 92.71) (width 0.25) (layer B.Cu) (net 20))
 (segment (start 194.31 98.425) (end 190.5 94.615) (width 0.25) (layer B.Cu) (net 20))
 (segment (start 194.31 100.965) (end 194.31 98.425) (width 0.25) (layer B.Cu) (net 20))
 (segment (start 193.675 101.6) (end 194.31 100.965) (width 0.25) (layer B.Cu) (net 20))
 (segment (start 189.865 101.6) (end 193.675 101.6) (width 0.25) (layer B.Cu) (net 20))
 (segment (start 171.45 105.41) (end 171.45 104.775) (width 0.25) (layer F.Cu) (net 20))
 (segment (start 171.45 104.775) (end 173.355 102.87) (width 0.25) (layer F.Cu) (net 20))
 (segment (start 173.355 102.87) (end 189.23 102.87) (width 0.25) (layer F.Cu) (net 20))
 (segment (start 177.8 92.71) (end 177.8 92.075) (width 0.25) (layer F.Cu) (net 20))
 (segment (start 189.23 94.615) (end 190.5 93.345) (width 0.25) (layer F.Cu) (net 20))
 (segment (start 190.5 93.345) (end 190.5 92.71) (width 0.25) (layer F.Cu) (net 20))
 (segment (start 189.23 102.87) (end 188.595 102.87) (width 0.25) (layer F.Cu) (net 20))
 (segment (start 196.85 107.315) (end 200.025 104.14) (width 0.25) (layer B.Cu) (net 21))
 (segment (start 189.23 110.49) (end 189.23 109.22) (width 0.25) (layer B.Cu) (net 21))
 (segment (start 200.025 94.615) (end 198.12 92.71) (width 0.25) (layer B.Cu) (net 21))
 (segment (start 200.025 104.14) (end 200.025 94.615) (width 0.25) (layer B.Cu) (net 21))
 (segment (start 191.135 107.315) (end 196.85 107.315) (width 0.25) (layer B.Cu) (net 21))
 (segment (start 189.23 109.22) (end 191.135 107.315) (width 0.25) (layer B.Cu) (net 21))
 (segment (start 185.42 100.33) (end 185.42 104.14) (width 0.25) (layer B.Cu) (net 24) (status 20))
 (segment (start 185.42 104.14) (end 184.785 104.775) (width 0.25) (layer B.Cu) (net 24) (status 30))
 (segment (start 180.975 107.95) (end 194.31 107.95) (width 0.25) (layer F.Cu) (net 24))
 (segment (start 194.31 107.95) (end 196.85 110.49) (width 0.25) (layer F.Cu) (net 24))
 (segment (start 184.785 104.775) (end 180.975 107.95) (width 0.25) (layer F.Cu) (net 24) (status 10))
 (segment (start 180.975 107.95) (end 171.45 107.95) (width 0.25) (layer F.Cu) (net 24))
 (segment (start 184.15 105.41) (end 184.785 104.775) (width 0.25) (layer F.Cu) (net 24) (status 30))
 (segment (start 184.785 104.775) (end 185.42 104.14) (width 0.25) (layer B.Cu) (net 24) (status 30))
 (segment (start 177.165 104.775) (end 179.705 104.775) (width 0.25) (layer B.Cu) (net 25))
 (segment (start 182.88 101.6) (end 182.88 100.33) (width 0.25) (layer B.Cu) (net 25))
 (segment (start 179.705 104.775) (end 182.88 101.6) (width 0.25) (layer B.Cu) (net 25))
 (segment (start 182.88 100.33) (end 182.88 100.965) (width 0.25) (layer B.Cu) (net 25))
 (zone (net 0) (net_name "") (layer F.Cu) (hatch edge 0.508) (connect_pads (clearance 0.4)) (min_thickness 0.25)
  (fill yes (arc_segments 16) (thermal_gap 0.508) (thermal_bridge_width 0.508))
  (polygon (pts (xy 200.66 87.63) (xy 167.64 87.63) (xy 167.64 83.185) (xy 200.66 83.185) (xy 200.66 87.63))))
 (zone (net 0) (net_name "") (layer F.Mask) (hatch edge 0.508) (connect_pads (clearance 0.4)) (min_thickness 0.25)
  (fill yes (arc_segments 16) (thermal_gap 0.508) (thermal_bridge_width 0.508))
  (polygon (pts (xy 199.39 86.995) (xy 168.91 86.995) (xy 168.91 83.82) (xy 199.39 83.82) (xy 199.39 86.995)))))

